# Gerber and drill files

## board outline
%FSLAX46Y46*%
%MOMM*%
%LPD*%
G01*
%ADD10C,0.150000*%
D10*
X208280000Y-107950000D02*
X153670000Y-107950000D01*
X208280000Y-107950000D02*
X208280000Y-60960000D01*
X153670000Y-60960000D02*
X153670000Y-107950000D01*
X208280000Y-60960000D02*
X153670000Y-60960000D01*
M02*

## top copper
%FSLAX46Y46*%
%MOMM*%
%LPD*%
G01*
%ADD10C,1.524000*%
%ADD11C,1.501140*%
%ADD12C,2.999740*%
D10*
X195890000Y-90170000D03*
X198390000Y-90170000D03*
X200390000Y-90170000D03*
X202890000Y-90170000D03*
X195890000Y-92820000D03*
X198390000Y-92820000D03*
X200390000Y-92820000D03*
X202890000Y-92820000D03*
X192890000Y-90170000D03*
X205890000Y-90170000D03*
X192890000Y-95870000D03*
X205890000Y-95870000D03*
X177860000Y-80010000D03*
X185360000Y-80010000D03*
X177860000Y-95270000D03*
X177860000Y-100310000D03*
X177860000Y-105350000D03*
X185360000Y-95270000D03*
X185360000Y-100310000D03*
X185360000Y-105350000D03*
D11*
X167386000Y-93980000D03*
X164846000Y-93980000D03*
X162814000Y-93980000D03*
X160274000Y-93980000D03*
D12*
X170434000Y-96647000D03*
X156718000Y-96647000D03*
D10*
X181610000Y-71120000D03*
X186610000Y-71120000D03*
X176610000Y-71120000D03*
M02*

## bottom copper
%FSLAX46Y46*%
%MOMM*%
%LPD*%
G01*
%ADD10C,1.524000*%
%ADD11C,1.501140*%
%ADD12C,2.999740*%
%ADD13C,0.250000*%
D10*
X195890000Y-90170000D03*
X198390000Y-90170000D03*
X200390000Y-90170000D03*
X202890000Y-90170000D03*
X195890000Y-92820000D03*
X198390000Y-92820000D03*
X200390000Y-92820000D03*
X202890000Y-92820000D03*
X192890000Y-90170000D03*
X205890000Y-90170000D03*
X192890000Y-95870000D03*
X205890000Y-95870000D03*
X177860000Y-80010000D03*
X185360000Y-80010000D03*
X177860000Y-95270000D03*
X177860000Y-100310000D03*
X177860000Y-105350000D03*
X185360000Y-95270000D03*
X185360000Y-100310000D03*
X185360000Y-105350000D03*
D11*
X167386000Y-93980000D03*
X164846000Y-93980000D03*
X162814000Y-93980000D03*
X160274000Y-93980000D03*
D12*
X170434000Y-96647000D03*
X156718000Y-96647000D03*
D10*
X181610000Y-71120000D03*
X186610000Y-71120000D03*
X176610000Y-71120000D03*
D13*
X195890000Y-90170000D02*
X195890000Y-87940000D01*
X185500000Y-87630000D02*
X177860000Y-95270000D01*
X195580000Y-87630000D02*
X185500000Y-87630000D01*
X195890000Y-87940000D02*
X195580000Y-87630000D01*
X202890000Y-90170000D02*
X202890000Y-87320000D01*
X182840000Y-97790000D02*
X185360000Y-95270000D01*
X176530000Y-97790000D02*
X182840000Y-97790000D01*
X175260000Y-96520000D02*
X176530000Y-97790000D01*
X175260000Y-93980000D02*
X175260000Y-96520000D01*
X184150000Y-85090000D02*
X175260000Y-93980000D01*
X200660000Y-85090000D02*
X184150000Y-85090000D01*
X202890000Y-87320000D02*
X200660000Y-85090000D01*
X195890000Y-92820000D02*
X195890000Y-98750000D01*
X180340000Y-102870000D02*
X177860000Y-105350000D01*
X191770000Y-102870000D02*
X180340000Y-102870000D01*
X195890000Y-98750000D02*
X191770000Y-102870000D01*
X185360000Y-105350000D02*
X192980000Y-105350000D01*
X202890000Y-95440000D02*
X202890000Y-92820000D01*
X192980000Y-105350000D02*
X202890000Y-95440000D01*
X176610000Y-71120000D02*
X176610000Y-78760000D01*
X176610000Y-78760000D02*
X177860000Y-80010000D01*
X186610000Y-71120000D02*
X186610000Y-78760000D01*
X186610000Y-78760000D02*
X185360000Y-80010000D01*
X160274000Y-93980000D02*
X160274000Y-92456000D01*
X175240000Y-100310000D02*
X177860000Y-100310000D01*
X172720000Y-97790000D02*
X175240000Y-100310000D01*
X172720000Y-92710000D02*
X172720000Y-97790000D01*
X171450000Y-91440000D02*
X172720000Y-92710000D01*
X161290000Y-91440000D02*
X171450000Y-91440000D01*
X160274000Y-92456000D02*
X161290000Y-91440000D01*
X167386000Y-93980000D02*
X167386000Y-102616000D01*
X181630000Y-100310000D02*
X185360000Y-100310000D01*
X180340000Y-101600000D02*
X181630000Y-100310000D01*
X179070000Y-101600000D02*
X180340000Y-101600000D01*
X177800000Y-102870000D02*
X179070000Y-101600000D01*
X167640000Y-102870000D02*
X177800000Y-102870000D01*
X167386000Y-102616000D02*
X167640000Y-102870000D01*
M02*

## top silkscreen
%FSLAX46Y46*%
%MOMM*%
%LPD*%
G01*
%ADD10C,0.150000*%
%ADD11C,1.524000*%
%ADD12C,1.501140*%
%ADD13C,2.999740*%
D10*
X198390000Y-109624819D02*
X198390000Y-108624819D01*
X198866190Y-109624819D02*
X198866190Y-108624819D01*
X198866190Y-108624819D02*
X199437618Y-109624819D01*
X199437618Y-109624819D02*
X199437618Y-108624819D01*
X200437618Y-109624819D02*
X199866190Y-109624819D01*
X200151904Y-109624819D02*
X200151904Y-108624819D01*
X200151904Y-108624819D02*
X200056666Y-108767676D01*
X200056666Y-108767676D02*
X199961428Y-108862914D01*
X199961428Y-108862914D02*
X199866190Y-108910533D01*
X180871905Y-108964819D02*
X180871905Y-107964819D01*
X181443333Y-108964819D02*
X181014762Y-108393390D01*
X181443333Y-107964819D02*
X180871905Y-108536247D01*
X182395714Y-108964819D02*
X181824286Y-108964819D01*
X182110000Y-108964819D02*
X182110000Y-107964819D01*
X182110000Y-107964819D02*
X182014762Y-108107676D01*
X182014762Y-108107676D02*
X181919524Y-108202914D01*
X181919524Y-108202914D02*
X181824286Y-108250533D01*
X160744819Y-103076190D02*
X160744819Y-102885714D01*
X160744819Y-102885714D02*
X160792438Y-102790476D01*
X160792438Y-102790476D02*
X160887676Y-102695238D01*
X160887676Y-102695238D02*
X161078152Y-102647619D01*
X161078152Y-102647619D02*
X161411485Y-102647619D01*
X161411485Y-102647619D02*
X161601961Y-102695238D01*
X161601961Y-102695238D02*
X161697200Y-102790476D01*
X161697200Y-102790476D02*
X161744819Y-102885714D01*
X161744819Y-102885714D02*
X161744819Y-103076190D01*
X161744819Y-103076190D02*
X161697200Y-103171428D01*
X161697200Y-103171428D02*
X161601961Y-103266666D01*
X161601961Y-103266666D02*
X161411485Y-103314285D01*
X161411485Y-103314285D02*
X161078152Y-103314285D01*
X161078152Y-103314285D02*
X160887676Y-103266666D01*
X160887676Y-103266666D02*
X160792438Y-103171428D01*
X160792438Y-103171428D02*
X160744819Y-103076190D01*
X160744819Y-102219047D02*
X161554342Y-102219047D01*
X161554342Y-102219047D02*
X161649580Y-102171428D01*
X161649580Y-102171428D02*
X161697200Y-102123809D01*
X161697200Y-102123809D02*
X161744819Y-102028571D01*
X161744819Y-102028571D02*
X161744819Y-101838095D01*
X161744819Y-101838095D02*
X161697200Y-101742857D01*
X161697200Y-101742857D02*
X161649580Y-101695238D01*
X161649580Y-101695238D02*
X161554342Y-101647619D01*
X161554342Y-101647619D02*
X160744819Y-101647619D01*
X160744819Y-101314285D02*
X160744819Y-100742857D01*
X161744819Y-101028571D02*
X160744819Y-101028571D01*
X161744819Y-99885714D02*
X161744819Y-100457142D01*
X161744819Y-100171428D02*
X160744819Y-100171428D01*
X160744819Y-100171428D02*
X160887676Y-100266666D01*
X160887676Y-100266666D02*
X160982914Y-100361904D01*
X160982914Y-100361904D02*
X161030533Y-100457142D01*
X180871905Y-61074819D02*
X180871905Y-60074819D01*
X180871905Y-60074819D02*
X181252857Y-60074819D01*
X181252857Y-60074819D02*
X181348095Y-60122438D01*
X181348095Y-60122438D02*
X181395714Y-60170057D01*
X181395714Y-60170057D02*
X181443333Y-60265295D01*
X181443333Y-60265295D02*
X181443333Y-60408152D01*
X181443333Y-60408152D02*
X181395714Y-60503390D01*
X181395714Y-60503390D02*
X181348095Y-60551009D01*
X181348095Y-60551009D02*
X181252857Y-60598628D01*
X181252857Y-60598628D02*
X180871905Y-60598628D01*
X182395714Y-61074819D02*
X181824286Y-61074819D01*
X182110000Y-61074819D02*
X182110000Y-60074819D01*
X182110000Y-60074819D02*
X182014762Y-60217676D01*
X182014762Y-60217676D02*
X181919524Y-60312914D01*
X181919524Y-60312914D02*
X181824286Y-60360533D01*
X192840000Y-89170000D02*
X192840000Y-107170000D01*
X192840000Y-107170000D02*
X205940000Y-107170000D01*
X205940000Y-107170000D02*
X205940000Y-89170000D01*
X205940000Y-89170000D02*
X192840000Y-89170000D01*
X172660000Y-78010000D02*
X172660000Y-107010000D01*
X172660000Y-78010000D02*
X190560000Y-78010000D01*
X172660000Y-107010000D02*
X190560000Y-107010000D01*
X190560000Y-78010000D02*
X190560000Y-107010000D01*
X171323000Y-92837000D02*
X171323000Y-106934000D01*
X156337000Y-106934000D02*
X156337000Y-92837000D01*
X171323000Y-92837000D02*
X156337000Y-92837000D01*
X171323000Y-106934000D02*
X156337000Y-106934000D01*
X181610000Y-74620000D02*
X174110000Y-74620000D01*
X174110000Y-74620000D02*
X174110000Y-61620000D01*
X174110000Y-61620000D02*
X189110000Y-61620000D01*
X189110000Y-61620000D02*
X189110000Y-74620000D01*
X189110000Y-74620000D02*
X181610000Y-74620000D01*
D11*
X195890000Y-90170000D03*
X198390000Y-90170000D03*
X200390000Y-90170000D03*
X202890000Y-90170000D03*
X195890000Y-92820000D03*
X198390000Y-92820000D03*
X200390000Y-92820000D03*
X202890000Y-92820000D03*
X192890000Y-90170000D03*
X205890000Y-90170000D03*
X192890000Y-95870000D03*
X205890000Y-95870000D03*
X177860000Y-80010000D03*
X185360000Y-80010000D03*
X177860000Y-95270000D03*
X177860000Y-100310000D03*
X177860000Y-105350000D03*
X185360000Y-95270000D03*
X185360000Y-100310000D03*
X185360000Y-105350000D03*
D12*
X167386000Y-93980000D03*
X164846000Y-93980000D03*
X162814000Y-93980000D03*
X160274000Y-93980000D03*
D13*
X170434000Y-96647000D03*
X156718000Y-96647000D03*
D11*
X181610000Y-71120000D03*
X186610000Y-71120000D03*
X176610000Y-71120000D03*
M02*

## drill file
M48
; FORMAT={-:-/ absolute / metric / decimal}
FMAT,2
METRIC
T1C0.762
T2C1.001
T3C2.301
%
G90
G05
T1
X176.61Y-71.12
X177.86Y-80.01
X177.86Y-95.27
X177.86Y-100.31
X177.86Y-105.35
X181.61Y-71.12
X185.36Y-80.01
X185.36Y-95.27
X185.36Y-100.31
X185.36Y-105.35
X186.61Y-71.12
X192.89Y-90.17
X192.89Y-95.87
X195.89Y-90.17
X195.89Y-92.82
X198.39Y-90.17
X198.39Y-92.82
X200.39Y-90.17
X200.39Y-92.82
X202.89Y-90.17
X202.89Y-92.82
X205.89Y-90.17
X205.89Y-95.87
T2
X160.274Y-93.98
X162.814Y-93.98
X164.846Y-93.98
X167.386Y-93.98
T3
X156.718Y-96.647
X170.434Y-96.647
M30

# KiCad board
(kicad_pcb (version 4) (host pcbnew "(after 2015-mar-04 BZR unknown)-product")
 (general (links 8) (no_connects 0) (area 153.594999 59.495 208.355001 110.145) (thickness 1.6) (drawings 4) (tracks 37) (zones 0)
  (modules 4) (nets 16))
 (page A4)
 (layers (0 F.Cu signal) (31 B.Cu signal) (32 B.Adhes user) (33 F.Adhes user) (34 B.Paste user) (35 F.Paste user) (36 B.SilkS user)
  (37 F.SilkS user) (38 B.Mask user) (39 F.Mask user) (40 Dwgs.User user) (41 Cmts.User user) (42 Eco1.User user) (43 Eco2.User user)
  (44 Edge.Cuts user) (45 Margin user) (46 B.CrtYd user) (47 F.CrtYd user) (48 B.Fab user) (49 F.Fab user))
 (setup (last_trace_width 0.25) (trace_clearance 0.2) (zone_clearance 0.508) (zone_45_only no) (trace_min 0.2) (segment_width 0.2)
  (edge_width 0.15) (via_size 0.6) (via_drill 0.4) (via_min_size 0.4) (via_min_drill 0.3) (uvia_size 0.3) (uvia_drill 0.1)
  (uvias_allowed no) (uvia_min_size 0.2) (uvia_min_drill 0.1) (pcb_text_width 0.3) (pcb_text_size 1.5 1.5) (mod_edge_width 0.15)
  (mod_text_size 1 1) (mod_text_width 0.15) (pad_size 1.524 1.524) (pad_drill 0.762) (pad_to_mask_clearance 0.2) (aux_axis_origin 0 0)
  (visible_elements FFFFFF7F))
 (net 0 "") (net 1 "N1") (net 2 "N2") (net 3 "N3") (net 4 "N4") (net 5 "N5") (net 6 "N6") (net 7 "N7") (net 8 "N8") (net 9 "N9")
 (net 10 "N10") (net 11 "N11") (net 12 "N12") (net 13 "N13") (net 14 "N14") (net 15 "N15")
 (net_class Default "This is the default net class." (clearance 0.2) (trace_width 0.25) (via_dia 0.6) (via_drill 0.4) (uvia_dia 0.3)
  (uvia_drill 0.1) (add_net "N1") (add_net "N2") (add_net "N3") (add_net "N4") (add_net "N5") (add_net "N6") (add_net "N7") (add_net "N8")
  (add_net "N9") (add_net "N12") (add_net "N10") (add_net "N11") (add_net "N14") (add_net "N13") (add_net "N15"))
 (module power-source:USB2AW (layer F.Cu) (at 199.39 90.17)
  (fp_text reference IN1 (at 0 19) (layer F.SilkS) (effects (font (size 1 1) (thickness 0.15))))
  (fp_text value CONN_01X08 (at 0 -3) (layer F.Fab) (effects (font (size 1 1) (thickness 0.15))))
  (fp_line (start -6.55 -1) (end -6.55 17) (layer F.SilkS) (width 0.15))
  (fp_line (start -6.55 17) (end 6.55 17) (layer F.SilkS) (width 0.15))
  (fp_line (start 6.55 17) (end 6.55 -1) (layer F.SilkS) (width 0.15))
  (fp_line (start 6.55 -1) (end -6.55 -1) (layer F.SilkS) (width 0.15))
  (pad 1 thru_hole circle (at -3.5 0) (size 1.524 1.524) (drill 0.762) (layers *.Cu *.Mask F.SilkS) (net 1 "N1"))
  (pad 2 thru_hole circle (at -1 0) (size 1.524 1.524) (drill 0.762) (layers *.Cu *.Mask F.SilkS) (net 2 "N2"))
  (pad 3 thru_hole circle (at 1 0) (size 1.524 1.524) (drill 0.762) (layers *.Cu *.Mask F.SilkS) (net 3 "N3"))
  (pad 4 thru_hole circle (at 3.5 0) (size 1.524 1.524) (drill 0.762) (layers *.Cu *.Mask F.SilkS) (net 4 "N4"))
  (pad 5 thru_hole circle (at -3.5 2.65) (size 1.524 1.524) (drill 0.762) (layers *.Cu *.Mask F.SilkS) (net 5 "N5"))
  (pad 6 thru_hole circle (at -1 2.65) (size 1.524 1.524) (drill 0.762) (layers *.Cu *.Mask F.SilkS) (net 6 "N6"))
  (pad 7 thru_hole circle (at 1 2.65) (size 1.524 1.524) (drill 0.762) (layers *.Cu *.Mask F.SilkS) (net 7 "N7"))
  (pad 8 thru_hole circle (at 3.5 2.65) (size 1.524 1.524) (drill 0.762) (layers *.Cu *.Mask F.SilkS) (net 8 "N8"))
  (pad 14 thru_hole circle (at -6.5 0) (size 1.524 1.524) (drill 0.762) (layers *.Cu *.Mask F.SilkS))
  (pad 15 thru_hole circle (at 6.5 0) (size 1.524 1.524) (drill 0.762) (layers *.Cu *.Mask F.SilkS))
  (pad 16 thru_hole circle (at -6.5 5.7) (size 1.524 1.524) (drill 0.762) (layers *.Cu *.Mask F.SilkS))
  (pad 17 thru_hole circle (at 6.5 5.7) (size 1.524 1.524) (drill 0.762) (layers *.Cu *.Mask F.SilkS)))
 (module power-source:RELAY (layer F.Cu) (at 181.61 80.01)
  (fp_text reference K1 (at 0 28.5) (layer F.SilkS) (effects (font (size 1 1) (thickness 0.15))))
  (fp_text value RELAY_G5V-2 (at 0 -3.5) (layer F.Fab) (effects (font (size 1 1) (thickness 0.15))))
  (fp_line (start -8.95 -2) (end -8.95 27) (layer F.SilkS) (width 0.15))
  (fp_line (start -8.95 -2) (end 8.95 -2) (layer F.SilkS) (width 0.15))
  (fp_line (start -8.95 27) (end 8.95 27) (layer F.SilkS) (width 0.15))
  (fp_line (start 8.95 -2) (end 8.95 27) (layer F.SilkS) (width 0.15))
  (pad 1 thru_hole circle (at -3.75 0) (size 1.524 1.524) (drill 0.762) (layers *.Cu *.Mask F.SilkS) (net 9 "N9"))
  (pad 16 thru_hole circle (at 3.75 0) (size 1.524 1.524) (drill 0.762) (layers *.Cu *.Mask F.SilkS) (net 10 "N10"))
  (pad 6 thru_hole circle (at -3.75 15.26) (size 1.524 1.524) (drill 0.762) (layers *.Cu *.Mask F.SilkS) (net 1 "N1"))
  (pad 4 thru_hole circle (at -3.75 20.3) (size 1.524 1.524) (drill 0.762) (layers *.Cu *.Mask F.SilkS) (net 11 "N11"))
  (pad 8 thru_hole circle (at -3.75 25.34) (size 1.524 1.524) (drill 0.762) (layers *.Cu *.Mask F.SilkS) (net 5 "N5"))
  (pad 11 thru_hole circle (at 3.75 15.26) (size 1.524 1.524) (drill 0.762) (layers *.Cu *.Mask F.SilkS) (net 4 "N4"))
  (pad 13 thru_hole circle (at 3.75 20.3) (size 1.524 1.524) (drill 0.762) (layers *.Cu *.Mask F.SilkS) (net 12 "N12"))
  (pad 9 thru_hole circle (at 3.75 25.34) (size 1.524 1.524) (drill 0.762) (layers *.Cu *.Mask F.SilkS) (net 8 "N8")))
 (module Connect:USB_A (layer F.Cu) (at 163.83 93.98 270)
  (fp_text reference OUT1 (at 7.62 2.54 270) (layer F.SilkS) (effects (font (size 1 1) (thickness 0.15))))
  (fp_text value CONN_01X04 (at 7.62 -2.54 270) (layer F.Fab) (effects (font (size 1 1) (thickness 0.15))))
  (fp_line (start -1.143 -7.493) (end 12.954 -7.493) (layer F.SilkS) (width 0.15))
  (fp_line (start 12.954 7.493) (end -1.143 7.493) (layer F.SilkS) (width 0.15))
  (fp_line (start -1.143 -7.493) (end -1.143 7.493) (layer F.SilkS) (width 0.15))
  (fp_line (start 12.954 -7.493) (end 12.954 7.493) (layer F.SilkS) (width 0.15))
  (pad 4 thru_hole circle (at 0 -3.556 270) (size 1.50114 1.50114) (drill 1.00076) (layers *.Cu *.Mask F.SilkS) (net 12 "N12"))
  (pad 3 thru_hole circle (at 0 -1.016 270) (size 1.50114 1.50114) (drill 1.00076) (layers *.Cu *.Mask F.SilkS) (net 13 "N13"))
  (pad 2 thru_hole circle (at 0 1.016 270) (size 1.50114 1.50114) (drill 1.00076) (layers *.Cu *.Mask F.SilkS) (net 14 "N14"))
  (pad 1 thru_hole circle (at 0 3.556 270) (size 1.50114 1.50114) (drill 1.00076) (layers *.Cu *.Mask F.SilkS) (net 11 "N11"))
  (pad 5 thru_hole circle (at 2.667 -6.604 270) (size 2.99974 2.99974) (drill 2.30124) (layers *.Cu *.Mask F.SilkS))
  (pad 6 thru_hole circle (at 2.667 7.112 270) (size 2.99974 2.99974) (drill 2.30124) (layers *.Cu *.Mask F.SilkS)))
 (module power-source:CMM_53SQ (layer F.Cu) (at 181.61 71.12 180)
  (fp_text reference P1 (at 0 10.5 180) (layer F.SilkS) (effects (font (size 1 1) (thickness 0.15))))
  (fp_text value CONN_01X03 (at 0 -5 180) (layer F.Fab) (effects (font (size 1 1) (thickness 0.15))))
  (fp_line (start 0 -3.5) (end 7.5 -3.5) (layer F.SilkS) (width 0.15))
  (fp_line (start 7.5 -3.5) (end 7.5 9.5) (layer F.SilkS) (width 0.15))
  (fp_line (start 7.5 9.5) (end -7.5 9.5) (layer F.SilkS) (width 0.15))
  (fp_line (start -7.5 9.5) (end -7.5 -3.5) (layer F.SilkS) (width 0.15))
  (fp_line (start -7.5 -3.5) (end 0 -3.5) (layer F.SilkS) (width 0.15))
  (pad 2 thru_hole circle (at 0 0 180) (size 1.524 1.524) (drill 0.762) (layers *.Cu *.Mask F.SilkS) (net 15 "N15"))
  (pad 1 thru_hole circle (at -5 0 180) (size 1.524 1.524) (drill 0.762) (layers *.Cu *.Mask F.SilkS) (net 10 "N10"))
  (pad 3 thru_hole circle (at 5 0 180) (size 1.524 1.524) (drill 0.762) (layers *.Cu *.Mask F.SilkS) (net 9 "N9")))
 (gr_line (start 208.28 107.95) (end 153.67 107.95) (angle 90) (layer Edge.Cuts) (width 0.15))
 (gr_line (start 208.28 107.95) (end 208.28 60.96) (angle 90) (layer Edge.Cuts) (width 0.15))
 (gr_line (start 153.67 60.96) (end 153.67 107.95) (angle 90) (layer Edge.Cuts) (width 0.15))
 (gr_line (start 208.28 60.96) (end 153.67 60.96) (angle 90) (layer Edge.Cuts) (width 0.15))
 (segment (start 195.89 90.17) (end 195.89 87.94) (width 0.25) (layer B.Cu) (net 1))
 (segment (start 185.5 87.63) (end 177.86 95.27) (width 0.25) (layer B.Cu) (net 1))
 (segment (start 195.58 87.63) (end 185.5 87.63) (width 0.25) (layer B.Cu) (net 1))
 (segment (start 195.89 87.94) (end 195.58 87.63) (width 0.25) (layer B.Cu) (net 1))
 (segment (start 202.89 90.17) (end 202.89 87.32) (width 0.25) (layer B.Cu) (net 4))
 (segment (start 182.84 97.79) (end 185.36 95.27) (width 0.25) (layer B.Cu) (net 4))
 (segment (start 176.53 97.79) (end 182.84 97.79) (width 0.25) (layer B.Cu) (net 4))
 (segment (start 175.26 96.52) (end 176.53 97.79) (width 0.25) (layer B.Cu) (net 4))
 (segment (start 175.26 93.98) (end 175.26 96.52) (width 0.25) (layer B.Cu) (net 4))
 (segment (start 184.15 85.09) (end 175.26 93.98) (width 0.25) (layer B.Cu) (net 4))
 (segment (start 200.66 85.09) (end 184.15 85.09) (width 0.25) (layer B.Cu) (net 4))
 (segment (start 202.89 87.32) (end 200.66 85.09) (width 0.25) (layer B.Cu) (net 4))
 (segment (start 195.89 92.82) (end 195.89 98.75) (width 0.25) (layer B.Cu) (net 5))
 (segment (start 180.34 102.87) (end 177.86 105.35) (width 0.25) (layer B.Cu) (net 5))
 (segment (start 191.77 102.87) (end 180.34 102.87) (width 0.25) (layer B.Cu) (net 5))
 (segment (start 195.89 98.75) (end 191.77 102.87) (width 0.25) (layer B.Cu) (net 5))
 (segment (start 185.36 105.35) (end 192.98 105.35) (width 0.25) (layer B.Cu) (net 8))
 (segment (start 202.89 95.44) (end 202.89 92.82) (width 0.25) (layer B.Cu) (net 8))
 (segment (start 192.98 105.35) (end 202.89 95.44) (width 0.25) (layer B.Cu) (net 8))
 (segment (start 176.61 71.12) (end 176.61 78.76) (width 0.25) (layer B.Cu) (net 9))
 (segment (start 176.61 78.76) (end 177.86 80.01) (width 0.25) (layer B.Cu) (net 9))
 (segment (start 186.61 71.12) (end 186.61 78.76) (width 0.25) (layer B.Cu) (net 10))
 (segment (start 186.61 78.76) (end 185.36 80.01) (width 0.25) (layer B.Cu) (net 10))
 (segment (start 160.274 93.98) (end 160.274 92.456) (width 0.25) (layer B.Cu) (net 11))
 (segment (start 175.24 100.31) (end 177.86 100.31) (width 0.25) (layer B.Cu) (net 11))
 (segment (start 172.72 97.79) (end 175.24 100.31) (width 0.25) (layer B.Cu) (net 11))
 (segment (start 172.72 92.71) (end 172.72 97.79) (width 0.25) (layer B.Cu) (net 11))
 (segment (start 171.45 91.44) (end 172.72 92.71) (width 0.25) (layer B.Cu) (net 11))
 (segment (start 161.29 91.44) (end 171.45 91.44) (width 0.25) (layer B.Cu) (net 11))
 (segment (start 160.274 92.456) (end 161.29 91.44) (width 0.25) (layer B.Cu) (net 11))
 (segment (start 167.386 93.98) (end 167.386 102.616) (width 0.25) (layer B.Cu) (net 12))
 (segment (start 181.63 100.31) (end 185.36 100.31) (width 0.25) (layer B.Cu) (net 12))
 (segment (start 180.34 101.6) (end 181.63 100.31) (width 0.25) (layer B.Cu) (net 12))
 (segment (start 179.07 101.6) (end 180.34 101.6) (width 0.25) (layer B.Cu) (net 12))
 (segment (start 177.8 102.87) (end 179.07 101.6) (width 0.25) (layer B.Cu) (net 12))
 (segment (start 167.64 102.87) (end 177.8 102.87) (width 0.25) (layer B.Cu) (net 12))
 (segment (start 167.386 102.616) (end 167.64 102.87) (width 0.25) (layer B.Cu) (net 12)))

